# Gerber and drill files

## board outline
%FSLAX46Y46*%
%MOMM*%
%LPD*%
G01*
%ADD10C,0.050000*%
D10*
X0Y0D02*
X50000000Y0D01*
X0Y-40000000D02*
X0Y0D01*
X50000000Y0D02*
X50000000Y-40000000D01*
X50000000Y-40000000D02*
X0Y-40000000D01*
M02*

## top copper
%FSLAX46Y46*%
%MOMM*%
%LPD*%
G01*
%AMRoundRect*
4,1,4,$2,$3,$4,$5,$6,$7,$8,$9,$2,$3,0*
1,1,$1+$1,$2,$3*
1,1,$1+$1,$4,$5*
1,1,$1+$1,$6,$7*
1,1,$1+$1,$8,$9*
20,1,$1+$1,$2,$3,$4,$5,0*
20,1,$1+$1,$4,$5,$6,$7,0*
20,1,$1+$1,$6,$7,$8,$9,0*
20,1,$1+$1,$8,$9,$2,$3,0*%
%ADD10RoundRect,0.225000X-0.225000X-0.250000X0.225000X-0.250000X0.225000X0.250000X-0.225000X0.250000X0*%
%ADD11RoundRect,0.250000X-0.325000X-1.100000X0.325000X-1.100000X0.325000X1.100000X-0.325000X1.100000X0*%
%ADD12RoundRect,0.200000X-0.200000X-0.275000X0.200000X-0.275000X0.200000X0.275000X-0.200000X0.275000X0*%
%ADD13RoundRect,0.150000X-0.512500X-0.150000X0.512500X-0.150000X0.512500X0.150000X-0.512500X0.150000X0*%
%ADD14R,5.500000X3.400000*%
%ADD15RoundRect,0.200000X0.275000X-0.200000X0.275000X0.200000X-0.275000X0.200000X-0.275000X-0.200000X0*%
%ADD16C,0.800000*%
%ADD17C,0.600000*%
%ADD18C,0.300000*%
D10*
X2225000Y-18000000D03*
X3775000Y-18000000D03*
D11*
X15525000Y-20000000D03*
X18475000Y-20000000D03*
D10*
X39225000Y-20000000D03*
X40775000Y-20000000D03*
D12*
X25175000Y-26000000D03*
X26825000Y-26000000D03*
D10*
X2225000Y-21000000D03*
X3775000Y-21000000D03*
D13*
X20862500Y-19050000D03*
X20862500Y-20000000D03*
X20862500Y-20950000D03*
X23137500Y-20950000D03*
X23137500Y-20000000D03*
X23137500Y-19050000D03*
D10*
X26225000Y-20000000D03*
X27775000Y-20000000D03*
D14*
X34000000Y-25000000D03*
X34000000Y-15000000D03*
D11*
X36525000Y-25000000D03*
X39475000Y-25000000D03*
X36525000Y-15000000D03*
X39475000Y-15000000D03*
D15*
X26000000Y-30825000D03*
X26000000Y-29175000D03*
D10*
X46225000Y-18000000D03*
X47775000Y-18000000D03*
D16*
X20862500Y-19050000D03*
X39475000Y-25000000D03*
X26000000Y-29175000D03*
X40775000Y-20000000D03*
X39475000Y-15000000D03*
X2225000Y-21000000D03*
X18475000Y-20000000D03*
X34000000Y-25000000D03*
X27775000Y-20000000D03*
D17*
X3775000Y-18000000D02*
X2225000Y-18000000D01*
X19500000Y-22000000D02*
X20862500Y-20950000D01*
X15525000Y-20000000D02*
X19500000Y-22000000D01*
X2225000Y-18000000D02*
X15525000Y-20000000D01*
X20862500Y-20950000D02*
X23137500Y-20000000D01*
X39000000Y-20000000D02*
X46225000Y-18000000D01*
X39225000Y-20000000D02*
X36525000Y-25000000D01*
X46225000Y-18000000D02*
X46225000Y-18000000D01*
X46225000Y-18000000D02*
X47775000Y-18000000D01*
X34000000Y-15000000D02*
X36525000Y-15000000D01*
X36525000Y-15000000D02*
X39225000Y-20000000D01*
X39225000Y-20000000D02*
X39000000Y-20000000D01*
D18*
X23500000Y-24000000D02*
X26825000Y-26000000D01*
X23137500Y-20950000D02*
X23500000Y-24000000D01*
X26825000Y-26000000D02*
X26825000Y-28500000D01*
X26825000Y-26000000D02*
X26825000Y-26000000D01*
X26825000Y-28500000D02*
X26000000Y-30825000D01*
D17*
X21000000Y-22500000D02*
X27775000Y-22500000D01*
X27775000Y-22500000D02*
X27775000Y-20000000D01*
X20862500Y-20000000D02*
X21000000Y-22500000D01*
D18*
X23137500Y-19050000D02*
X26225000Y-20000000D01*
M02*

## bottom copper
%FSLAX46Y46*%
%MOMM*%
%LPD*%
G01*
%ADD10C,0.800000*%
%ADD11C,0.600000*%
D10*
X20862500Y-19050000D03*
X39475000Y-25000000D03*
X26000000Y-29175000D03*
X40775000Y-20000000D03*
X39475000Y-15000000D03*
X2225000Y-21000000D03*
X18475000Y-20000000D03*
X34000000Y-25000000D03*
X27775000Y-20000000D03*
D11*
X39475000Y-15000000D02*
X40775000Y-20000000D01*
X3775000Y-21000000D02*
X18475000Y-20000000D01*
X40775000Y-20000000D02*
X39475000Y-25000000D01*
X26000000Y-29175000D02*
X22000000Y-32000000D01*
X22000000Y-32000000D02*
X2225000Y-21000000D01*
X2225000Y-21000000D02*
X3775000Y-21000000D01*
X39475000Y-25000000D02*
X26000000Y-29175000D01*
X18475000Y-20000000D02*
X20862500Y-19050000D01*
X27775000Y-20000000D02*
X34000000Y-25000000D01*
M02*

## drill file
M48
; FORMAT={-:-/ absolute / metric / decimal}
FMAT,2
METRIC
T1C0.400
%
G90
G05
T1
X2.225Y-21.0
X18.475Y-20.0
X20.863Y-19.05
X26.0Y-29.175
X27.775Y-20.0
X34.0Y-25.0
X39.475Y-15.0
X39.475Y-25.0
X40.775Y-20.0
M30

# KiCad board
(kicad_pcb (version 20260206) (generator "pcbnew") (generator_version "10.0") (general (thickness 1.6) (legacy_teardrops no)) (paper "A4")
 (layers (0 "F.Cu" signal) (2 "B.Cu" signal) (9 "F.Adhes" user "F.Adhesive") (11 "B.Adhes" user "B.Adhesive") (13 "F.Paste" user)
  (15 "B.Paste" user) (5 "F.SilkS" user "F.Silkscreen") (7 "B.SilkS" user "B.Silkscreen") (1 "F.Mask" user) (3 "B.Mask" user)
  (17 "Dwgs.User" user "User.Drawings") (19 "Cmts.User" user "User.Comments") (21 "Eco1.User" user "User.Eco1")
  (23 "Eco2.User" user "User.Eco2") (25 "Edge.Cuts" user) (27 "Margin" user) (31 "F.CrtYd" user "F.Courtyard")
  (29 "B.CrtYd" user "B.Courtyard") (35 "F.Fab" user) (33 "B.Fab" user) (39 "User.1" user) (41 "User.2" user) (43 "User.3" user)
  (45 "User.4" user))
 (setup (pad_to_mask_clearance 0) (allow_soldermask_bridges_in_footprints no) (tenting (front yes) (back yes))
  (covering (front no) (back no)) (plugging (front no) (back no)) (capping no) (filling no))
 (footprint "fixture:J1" (layer "F.Cu") (at 3 18)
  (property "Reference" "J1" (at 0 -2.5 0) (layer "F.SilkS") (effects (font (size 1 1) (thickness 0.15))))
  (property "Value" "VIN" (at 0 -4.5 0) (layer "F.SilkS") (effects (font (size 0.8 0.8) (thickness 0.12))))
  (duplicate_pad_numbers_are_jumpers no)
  (pad "1" smd roundrect (at -0.775 0) (size 0.9 0.95) (layers "F.Cu" "F.Mask" "F.Paste") (roundrect_rratio 0.25) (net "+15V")
   (thermal_bridge_angle 45))
  (pad "2" smd roundrect (at 0.775 0) (size 0.9 0.95) (layers "F.Cu" "F.Mask" "F.Paste") (roundrect_rratio 0.25) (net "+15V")
   (thermal_bridge_angle 45)))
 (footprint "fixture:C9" (layer "F.Cu") (at 17 20)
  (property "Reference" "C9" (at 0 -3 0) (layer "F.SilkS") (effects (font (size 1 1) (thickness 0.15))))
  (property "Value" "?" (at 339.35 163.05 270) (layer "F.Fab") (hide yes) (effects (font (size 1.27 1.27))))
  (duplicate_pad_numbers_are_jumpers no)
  (pad "1" smd roundrect (at -1.475 0) (size 1.15 2.7) (layers "F.Cu" "F.Mask" "F.Paste") (roundrect_rratio 0.217391) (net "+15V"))
  (pad "2" smd roundrect (at 1.475 0) (size 1.15 2.7) (layers "F.Cu" "F.Mask" "F.Paste") (roundrect_rratio 0.217391) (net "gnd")))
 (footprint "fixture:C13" (layer "F.Cu") (at 40 20)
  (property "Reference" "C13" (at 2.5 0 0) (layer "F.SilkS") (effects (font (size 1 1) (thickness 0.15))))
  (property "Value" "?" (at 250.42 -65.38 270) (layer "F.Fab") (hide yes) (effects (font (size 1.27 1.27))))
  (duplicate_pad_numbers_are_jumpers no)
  (pad "1" smd roundrect (at -0.775 0) (size 0.9 0.95) (layers "F.Cu" "F.Mask" "F.Paste") (roundrect_rratio 0.25) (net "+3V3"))
  (pad "2" smd roundrect (at 0.775 0) (size 0.9 0.95) (layers "F.Cu" "F.Mask" "F.Paste") (roundrect_rratio 0.25) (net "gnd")))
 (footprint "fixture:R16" (layer "F.Cu") (at 26 26)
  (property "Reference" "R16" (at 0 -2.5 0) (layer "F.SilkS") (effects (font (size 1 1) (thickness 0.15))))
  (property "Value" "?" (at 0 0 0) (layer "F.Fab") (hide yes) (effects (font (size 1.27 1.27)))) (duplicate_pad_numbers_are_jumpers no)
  (pad "1" smd roundrect (at -0.825 0) (size 0.8 0.95) (layers "F.Cu" "F.Mask" "F.Paste") (roundrect_rratio 0.25) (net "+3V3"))
  (pad "2" smd roundrect (at 0.825 0) (size 0.8 0.95) (layers "F.Cu" "F.Mask" "F.Paste") (roundrect_rratio 0.25) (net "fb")))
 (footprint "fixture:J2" (layer "F.Cu") (at 3 21)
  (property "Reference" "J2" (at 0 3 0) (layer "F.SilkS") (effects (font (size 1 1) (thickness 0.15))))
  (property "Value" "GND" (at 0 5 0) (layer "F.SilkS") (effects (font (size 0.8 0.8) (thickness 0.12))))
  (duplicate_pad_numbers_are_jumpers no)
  (pad "1" smd roundrect (at -0.775 0) (size 0.9 0.95) (layers "F.Cu" "F.Mask" "F.Paste") (roundrect_rratio 0.25) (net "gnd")
   (thermal_bridge_angle 45))
  (pad "2" smd roundrect (at 0.775 0) (size 0.9 0.95) (layers "F.Cu" "F.Mask" "F.Paste") (roundrect_rratio 0.25) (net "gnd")
   (thermal_bridge_angle 45)))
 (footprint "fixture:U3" (layer "F.Cu") (at 22 20)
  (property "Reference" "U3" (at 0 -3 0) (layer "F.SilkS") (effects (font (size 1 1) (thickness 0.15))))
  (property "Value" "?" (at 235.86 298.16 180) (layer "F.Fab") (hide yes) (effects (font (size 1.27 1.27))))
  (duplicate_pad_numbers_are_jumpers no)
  (pad "1" smd roundrect (at -1.1375 -0.95) (size 1.325 0.6) (layers "F.Cu" "F.Mask" "F.Paste") (roundrect_rratio 0.25) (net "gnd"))
  (pad "2" smd roundrect (at -1.1375 0) (size 1.325 0.6) (layers "F.Cu" "F.Mask" "F.Paste") (roundrect_rratio 0.25) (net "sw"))
  (pad "3" smd roundrect (at -1.1375 0.95) (size 1.325 0.6) (layers "F.Cu" "F.Mask" "F.Paste") (roundrect_rratio 0.25) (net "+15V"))
  (pad "4" smd roundrect (at 1.1375 0.95) (size 1.325 0.6) (layers "F.Cu" "F.Mask" "F.Paste") (roundrect_rratio 0.25) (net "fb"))
  (pad "5" smd roundrect (at 1.1375 0) (size 1.325 0.6) (layers "F.Cu" "F.Mask" "F.Paste") (roundrect_rratio 0.25) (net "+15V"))
  (pad "6" smd roundrect (at 1.1375 -0.95) (size 1.325 0.6) (layers "F.Cu" "F.Mask" "F.Paste") (roundrect_rratio 0.25) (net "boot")))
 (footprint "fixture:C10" (layer "F.Cu") (at 27 20)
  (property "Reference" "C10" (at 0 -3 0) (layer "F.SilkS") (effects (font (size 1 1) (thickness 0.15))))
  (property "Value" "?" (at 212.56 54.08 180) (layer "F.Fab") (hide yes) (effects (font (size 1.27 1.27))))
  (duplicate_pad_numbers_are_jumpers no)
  (pad "1" smd roundrect (at -0.775 0) (size 0.9 0.95) (layers "F.Cu" "F.Mask" "F.Paste") (roundrect_rratio 0.25) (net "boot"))
  (pad "2" smd roundrect (at 0.775 0) (size 0.9 0.95) (layers "F.Cu" "F.Mask" "F.Paste") (roundrect_rratio 0.25) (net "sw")))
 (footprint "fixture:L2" (layer "F.Cu") (at 34 20 90)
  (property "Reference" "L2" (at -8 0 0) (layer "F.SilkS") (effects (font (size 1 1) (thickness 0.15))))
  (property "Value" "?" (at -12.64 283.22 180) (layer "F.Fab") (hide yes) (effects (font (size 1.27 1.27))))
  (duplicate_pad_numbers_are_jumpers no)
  (pad "1" smd rect (at -5 0 90) (size 3.4 5.5) (layers "F.Cu" "F.Mask" "F.Paste") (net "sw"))
  (pad "2" smd rect (at 5 0 90) (size 3.4 5.5) (layers "F.Cu" "F.Mask" "F.Paste") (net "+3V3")))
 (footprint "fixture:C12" (layer "F.Cu") (at 38 25)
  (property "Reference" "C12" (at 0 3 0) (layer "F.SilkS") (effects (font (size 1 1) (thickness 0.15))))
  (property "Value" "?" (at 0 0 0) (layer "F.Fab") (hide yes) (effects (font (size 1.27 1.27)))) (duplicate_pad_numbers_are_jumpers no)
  (pad "1" smd roundrect (at -1.475 0) (size 1.15 2.7) (layers "F.Cu" "F.Mask" "F.Paste") (roundrect_rratio 0.217391) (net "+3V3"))
  (pad "2" smd roundrect (at 1.475 0) (size 1.15 2.7) (layers "F.Cu" "F.Mask" "F.Paste") (roundrect_rratio 0.217391) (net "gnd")))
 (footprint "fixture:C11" (layer "F.Cu") (at 38 15)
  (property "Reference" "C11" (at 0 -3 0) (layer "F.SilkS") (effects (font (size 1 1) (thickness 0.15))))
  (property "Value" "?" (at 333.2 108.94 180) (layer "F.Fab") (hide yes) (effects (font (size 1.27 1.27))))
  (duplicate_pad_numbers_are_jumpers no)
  (pad "1" smd roundrect (at -1.475 0) (size 1.15 2.7) (layers "F.Cu" "F.Mask" "F.Paste") (roundrect_rratio 0.217391) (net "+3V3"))
  (pad "2" smd roundrect (at 1.475 0) (size 1.15 2.7) (layers "F.Cu" "F.Mask" "F.Paste") (roundrect_rratio 0.217391) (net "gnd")))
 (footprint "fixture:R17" (layer "F.Cu") (at 26 30 90)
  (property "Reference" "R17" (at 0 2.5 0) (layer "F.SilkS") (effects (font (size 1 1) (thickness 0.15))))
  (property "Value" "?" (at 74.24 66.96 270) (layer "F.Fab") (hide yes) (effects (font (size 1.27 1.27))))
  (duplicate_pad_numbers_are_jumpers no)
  (pad "1" smd roundrect (at -0.825 0 90) (size 0.8 0.95) (layers "F.Cu" "F.Mask" "F.Paste") (roundrect_rratio 0.25) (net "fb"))
  (pad "2" smd roundrect (at 0.825 0 90) (size 0.8 0.95) (layers "F.Cu" "F.Mask" "F.Paste") (roundrect_rratio 0.25) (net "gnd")))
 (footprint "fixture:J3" (layer "F.Cu") (at 47 18)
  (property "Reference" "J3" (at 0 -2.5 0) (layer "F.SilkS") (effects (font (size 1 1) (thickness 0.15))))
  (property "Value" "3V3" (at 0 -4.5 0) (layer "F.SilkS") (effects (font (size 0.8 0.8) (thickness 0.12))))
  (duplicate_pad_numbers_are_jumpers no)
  (pad "1" smd roundrect (at -0.775 0) (size 0.9 0.95) (layers "F.Cu" "F.Mask" "F.Paste") (roundrect_rratio 0.25) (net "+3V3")
   (thermal_bridge_angle 45))
  (pad "2" smd roundrect (at 0.775 0) (size 0.9 0.95) (layers "F.Cu" "F.Mask" "F.Paste") (roundrect_rratio 0.25) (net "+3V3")
   (thermal_bridge_angle 45)))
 (gr_line (start 0 0) (end 50 0) (stroke (width 0.05) (type default)) (layer "Edge.Cuts"))
 (gr_line (start 0 40) (end 0 0) (stroke (width 0.05) (type default)) (layer "Edge.Cuts"))
 (gr_line (start 50 0) (end 50 40) (stroke (width 0.05) (type default)) (layer "Edge.Cuts"))
 (gr_line (start 50 40) (end 0 40) (stroke (width 0.05) (type default)) (layer "Edge.Cuts"))
 (segment (start 3.775 18) (end 2.225 18) (width 0.6) (layer "F.Cu") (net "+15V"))
 (segment (start 19.5 22) (end 20.8625 20.95) (width 0.6) (layer "F.Cu") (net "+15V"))
 (segment (start 15.525 20) (end 19.5 22) (width 0.6) (layer "F.Cu") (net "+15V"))
 (segment (start 2.225 18) (end 15.525 20) (width 0.6) (layer "F.Cu") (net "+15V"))
 (segment (start 20.8625 20.95) (end 23.1375 20) (width 0.6) (layer "F.Cu") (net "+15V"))
 (via (at 20.8625 19.05) (size 0.8) (drill 0.4) (layers "F.Cu" "B.Cu") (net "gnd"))
 (via (at 39.475 25) (size 0.8) (drill 0.4) (layers "F.Cu" "B.Cu") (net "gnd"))
 (via (at 26 29.175) (size 0.8) (drill 0.4) (layers "F.Cu" "B.Cu") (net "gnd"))
 (via (at 40.775 20) (size 0.8) (drill 0.4) (layers "F.Cu" "B.Cu") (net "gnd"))
 (via (at 39.475 15) (size 0.8) (drill 0.4) (layers "F.Cu" "B.Cu") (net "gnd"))
 (via (at 2.225 21) (size 0.8) (drill 0.4) (layers "F.Cu" "B.Cu") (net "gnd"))
 (via (at 18.475 20) (size 0.8) (drill 0.4) (layers "F.Cu" "B.Cu") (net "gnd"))
 (segment (start 39.475 15) (end 40.775 20) (width 0.6) (layer "B.Cu") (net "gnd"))
 (segment (start 3.775 21) (end 18.475 20) (width 0.6) (layer "B.Cu") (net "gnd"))
 (segment (start 40.775 20) (end 39.475 25) (width 0.6) (layer "B.Cu") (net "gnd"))
 (segment (start 26 29.175) (end 22 32) (width 0.6) (layer "B.Cu") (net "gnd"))
 (segment (start 22 32) (end 2.225 21) (width 0.6) (layer "B.Cu") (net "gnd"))
 (segment (start 2.225 21) (end 3.775 21) (width 0.6) (layer "B.Cu") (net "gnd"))
 (segment (start 39.475 25) (end 26 29.175) (width 0.6) (layer "B.Cu") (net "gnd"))
 (segment (start 18.475 20) (end 20.8625 19.05) (width 0.6) (layer "B.Cu") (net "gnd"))
 (segment (start 39 20) (end 46.225 18) (width 0.6) (layer "F.Cu") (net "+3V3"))
 (segment (start 39.225 20) (end 36.525 25) (width 0.6) (layer "F.Cu") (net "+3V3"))
 (segment (start 46.225 18) (end 46.225 18) (width 0.6) (layer "F.Cu") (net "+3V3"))
 (segment (start 46.225 18) (end 47.775 18) (width 0.6) (layer "F.Cu") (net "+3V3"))
 (segment (start 34 15) (end 36.525 15) (width 0.6) (layer "F.Cu") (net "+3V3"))
 (segment (start 36.525 15) (end 39.225 20) (width 0.6) (layer "F.Cu") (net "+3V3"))
 (segment (start 39.225 20) (end 39 20) (width 0.6) (layer "F.Cu") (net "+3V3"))
 (segment (start 23.5 24) (end 26.825 26) (width 0.3) (layer "F.Cu") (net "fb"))
 (segment (start 23.1375 20.95) (end 23.5 24) (width 0.3) (layer "F.Cu") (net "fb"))
 (segment (start 26.825 26) (end 26.825 28.5) (width 0.3) (layer "F.Cu") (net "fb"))
 (segment (start 26.825 26) (end 26.825 26) (width 0.3) (layer "F.Cu") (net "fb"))
 (segment (start 26.825 28.5) (end 26 30.825) (width 0.3) (layer "F.Cu") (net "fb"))
 (segment (start 21 22.5) (end 27.775 22.5) (width 0.6) (layer "F.Cu") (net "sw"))
 (segment (start 27.775 22.5) (end 27.775 20) (width 0.6) (layer "F.Cu") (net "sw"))
 (segment (start 20.8625 20) (end 21 22.5) (width 0.6) (layer "F.Cu") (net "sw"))
 (via (at 34 25) (size 0.8) (drill 0.4) (layers "F.Cu" "B.Cu") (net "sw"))
 (via (at 27.775 20) (size 0.8) (drill 0.4) (layers "F.Cu" "B.Cu") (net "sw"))
 (segment (start 27.775 20) (end 34 25) (width 0.6) (layer "B.Cu") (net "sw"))
 (segment (start 23.1375 19.05) (end 26.225 20) (width 0.3) (layer "F.Cu") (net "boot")))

